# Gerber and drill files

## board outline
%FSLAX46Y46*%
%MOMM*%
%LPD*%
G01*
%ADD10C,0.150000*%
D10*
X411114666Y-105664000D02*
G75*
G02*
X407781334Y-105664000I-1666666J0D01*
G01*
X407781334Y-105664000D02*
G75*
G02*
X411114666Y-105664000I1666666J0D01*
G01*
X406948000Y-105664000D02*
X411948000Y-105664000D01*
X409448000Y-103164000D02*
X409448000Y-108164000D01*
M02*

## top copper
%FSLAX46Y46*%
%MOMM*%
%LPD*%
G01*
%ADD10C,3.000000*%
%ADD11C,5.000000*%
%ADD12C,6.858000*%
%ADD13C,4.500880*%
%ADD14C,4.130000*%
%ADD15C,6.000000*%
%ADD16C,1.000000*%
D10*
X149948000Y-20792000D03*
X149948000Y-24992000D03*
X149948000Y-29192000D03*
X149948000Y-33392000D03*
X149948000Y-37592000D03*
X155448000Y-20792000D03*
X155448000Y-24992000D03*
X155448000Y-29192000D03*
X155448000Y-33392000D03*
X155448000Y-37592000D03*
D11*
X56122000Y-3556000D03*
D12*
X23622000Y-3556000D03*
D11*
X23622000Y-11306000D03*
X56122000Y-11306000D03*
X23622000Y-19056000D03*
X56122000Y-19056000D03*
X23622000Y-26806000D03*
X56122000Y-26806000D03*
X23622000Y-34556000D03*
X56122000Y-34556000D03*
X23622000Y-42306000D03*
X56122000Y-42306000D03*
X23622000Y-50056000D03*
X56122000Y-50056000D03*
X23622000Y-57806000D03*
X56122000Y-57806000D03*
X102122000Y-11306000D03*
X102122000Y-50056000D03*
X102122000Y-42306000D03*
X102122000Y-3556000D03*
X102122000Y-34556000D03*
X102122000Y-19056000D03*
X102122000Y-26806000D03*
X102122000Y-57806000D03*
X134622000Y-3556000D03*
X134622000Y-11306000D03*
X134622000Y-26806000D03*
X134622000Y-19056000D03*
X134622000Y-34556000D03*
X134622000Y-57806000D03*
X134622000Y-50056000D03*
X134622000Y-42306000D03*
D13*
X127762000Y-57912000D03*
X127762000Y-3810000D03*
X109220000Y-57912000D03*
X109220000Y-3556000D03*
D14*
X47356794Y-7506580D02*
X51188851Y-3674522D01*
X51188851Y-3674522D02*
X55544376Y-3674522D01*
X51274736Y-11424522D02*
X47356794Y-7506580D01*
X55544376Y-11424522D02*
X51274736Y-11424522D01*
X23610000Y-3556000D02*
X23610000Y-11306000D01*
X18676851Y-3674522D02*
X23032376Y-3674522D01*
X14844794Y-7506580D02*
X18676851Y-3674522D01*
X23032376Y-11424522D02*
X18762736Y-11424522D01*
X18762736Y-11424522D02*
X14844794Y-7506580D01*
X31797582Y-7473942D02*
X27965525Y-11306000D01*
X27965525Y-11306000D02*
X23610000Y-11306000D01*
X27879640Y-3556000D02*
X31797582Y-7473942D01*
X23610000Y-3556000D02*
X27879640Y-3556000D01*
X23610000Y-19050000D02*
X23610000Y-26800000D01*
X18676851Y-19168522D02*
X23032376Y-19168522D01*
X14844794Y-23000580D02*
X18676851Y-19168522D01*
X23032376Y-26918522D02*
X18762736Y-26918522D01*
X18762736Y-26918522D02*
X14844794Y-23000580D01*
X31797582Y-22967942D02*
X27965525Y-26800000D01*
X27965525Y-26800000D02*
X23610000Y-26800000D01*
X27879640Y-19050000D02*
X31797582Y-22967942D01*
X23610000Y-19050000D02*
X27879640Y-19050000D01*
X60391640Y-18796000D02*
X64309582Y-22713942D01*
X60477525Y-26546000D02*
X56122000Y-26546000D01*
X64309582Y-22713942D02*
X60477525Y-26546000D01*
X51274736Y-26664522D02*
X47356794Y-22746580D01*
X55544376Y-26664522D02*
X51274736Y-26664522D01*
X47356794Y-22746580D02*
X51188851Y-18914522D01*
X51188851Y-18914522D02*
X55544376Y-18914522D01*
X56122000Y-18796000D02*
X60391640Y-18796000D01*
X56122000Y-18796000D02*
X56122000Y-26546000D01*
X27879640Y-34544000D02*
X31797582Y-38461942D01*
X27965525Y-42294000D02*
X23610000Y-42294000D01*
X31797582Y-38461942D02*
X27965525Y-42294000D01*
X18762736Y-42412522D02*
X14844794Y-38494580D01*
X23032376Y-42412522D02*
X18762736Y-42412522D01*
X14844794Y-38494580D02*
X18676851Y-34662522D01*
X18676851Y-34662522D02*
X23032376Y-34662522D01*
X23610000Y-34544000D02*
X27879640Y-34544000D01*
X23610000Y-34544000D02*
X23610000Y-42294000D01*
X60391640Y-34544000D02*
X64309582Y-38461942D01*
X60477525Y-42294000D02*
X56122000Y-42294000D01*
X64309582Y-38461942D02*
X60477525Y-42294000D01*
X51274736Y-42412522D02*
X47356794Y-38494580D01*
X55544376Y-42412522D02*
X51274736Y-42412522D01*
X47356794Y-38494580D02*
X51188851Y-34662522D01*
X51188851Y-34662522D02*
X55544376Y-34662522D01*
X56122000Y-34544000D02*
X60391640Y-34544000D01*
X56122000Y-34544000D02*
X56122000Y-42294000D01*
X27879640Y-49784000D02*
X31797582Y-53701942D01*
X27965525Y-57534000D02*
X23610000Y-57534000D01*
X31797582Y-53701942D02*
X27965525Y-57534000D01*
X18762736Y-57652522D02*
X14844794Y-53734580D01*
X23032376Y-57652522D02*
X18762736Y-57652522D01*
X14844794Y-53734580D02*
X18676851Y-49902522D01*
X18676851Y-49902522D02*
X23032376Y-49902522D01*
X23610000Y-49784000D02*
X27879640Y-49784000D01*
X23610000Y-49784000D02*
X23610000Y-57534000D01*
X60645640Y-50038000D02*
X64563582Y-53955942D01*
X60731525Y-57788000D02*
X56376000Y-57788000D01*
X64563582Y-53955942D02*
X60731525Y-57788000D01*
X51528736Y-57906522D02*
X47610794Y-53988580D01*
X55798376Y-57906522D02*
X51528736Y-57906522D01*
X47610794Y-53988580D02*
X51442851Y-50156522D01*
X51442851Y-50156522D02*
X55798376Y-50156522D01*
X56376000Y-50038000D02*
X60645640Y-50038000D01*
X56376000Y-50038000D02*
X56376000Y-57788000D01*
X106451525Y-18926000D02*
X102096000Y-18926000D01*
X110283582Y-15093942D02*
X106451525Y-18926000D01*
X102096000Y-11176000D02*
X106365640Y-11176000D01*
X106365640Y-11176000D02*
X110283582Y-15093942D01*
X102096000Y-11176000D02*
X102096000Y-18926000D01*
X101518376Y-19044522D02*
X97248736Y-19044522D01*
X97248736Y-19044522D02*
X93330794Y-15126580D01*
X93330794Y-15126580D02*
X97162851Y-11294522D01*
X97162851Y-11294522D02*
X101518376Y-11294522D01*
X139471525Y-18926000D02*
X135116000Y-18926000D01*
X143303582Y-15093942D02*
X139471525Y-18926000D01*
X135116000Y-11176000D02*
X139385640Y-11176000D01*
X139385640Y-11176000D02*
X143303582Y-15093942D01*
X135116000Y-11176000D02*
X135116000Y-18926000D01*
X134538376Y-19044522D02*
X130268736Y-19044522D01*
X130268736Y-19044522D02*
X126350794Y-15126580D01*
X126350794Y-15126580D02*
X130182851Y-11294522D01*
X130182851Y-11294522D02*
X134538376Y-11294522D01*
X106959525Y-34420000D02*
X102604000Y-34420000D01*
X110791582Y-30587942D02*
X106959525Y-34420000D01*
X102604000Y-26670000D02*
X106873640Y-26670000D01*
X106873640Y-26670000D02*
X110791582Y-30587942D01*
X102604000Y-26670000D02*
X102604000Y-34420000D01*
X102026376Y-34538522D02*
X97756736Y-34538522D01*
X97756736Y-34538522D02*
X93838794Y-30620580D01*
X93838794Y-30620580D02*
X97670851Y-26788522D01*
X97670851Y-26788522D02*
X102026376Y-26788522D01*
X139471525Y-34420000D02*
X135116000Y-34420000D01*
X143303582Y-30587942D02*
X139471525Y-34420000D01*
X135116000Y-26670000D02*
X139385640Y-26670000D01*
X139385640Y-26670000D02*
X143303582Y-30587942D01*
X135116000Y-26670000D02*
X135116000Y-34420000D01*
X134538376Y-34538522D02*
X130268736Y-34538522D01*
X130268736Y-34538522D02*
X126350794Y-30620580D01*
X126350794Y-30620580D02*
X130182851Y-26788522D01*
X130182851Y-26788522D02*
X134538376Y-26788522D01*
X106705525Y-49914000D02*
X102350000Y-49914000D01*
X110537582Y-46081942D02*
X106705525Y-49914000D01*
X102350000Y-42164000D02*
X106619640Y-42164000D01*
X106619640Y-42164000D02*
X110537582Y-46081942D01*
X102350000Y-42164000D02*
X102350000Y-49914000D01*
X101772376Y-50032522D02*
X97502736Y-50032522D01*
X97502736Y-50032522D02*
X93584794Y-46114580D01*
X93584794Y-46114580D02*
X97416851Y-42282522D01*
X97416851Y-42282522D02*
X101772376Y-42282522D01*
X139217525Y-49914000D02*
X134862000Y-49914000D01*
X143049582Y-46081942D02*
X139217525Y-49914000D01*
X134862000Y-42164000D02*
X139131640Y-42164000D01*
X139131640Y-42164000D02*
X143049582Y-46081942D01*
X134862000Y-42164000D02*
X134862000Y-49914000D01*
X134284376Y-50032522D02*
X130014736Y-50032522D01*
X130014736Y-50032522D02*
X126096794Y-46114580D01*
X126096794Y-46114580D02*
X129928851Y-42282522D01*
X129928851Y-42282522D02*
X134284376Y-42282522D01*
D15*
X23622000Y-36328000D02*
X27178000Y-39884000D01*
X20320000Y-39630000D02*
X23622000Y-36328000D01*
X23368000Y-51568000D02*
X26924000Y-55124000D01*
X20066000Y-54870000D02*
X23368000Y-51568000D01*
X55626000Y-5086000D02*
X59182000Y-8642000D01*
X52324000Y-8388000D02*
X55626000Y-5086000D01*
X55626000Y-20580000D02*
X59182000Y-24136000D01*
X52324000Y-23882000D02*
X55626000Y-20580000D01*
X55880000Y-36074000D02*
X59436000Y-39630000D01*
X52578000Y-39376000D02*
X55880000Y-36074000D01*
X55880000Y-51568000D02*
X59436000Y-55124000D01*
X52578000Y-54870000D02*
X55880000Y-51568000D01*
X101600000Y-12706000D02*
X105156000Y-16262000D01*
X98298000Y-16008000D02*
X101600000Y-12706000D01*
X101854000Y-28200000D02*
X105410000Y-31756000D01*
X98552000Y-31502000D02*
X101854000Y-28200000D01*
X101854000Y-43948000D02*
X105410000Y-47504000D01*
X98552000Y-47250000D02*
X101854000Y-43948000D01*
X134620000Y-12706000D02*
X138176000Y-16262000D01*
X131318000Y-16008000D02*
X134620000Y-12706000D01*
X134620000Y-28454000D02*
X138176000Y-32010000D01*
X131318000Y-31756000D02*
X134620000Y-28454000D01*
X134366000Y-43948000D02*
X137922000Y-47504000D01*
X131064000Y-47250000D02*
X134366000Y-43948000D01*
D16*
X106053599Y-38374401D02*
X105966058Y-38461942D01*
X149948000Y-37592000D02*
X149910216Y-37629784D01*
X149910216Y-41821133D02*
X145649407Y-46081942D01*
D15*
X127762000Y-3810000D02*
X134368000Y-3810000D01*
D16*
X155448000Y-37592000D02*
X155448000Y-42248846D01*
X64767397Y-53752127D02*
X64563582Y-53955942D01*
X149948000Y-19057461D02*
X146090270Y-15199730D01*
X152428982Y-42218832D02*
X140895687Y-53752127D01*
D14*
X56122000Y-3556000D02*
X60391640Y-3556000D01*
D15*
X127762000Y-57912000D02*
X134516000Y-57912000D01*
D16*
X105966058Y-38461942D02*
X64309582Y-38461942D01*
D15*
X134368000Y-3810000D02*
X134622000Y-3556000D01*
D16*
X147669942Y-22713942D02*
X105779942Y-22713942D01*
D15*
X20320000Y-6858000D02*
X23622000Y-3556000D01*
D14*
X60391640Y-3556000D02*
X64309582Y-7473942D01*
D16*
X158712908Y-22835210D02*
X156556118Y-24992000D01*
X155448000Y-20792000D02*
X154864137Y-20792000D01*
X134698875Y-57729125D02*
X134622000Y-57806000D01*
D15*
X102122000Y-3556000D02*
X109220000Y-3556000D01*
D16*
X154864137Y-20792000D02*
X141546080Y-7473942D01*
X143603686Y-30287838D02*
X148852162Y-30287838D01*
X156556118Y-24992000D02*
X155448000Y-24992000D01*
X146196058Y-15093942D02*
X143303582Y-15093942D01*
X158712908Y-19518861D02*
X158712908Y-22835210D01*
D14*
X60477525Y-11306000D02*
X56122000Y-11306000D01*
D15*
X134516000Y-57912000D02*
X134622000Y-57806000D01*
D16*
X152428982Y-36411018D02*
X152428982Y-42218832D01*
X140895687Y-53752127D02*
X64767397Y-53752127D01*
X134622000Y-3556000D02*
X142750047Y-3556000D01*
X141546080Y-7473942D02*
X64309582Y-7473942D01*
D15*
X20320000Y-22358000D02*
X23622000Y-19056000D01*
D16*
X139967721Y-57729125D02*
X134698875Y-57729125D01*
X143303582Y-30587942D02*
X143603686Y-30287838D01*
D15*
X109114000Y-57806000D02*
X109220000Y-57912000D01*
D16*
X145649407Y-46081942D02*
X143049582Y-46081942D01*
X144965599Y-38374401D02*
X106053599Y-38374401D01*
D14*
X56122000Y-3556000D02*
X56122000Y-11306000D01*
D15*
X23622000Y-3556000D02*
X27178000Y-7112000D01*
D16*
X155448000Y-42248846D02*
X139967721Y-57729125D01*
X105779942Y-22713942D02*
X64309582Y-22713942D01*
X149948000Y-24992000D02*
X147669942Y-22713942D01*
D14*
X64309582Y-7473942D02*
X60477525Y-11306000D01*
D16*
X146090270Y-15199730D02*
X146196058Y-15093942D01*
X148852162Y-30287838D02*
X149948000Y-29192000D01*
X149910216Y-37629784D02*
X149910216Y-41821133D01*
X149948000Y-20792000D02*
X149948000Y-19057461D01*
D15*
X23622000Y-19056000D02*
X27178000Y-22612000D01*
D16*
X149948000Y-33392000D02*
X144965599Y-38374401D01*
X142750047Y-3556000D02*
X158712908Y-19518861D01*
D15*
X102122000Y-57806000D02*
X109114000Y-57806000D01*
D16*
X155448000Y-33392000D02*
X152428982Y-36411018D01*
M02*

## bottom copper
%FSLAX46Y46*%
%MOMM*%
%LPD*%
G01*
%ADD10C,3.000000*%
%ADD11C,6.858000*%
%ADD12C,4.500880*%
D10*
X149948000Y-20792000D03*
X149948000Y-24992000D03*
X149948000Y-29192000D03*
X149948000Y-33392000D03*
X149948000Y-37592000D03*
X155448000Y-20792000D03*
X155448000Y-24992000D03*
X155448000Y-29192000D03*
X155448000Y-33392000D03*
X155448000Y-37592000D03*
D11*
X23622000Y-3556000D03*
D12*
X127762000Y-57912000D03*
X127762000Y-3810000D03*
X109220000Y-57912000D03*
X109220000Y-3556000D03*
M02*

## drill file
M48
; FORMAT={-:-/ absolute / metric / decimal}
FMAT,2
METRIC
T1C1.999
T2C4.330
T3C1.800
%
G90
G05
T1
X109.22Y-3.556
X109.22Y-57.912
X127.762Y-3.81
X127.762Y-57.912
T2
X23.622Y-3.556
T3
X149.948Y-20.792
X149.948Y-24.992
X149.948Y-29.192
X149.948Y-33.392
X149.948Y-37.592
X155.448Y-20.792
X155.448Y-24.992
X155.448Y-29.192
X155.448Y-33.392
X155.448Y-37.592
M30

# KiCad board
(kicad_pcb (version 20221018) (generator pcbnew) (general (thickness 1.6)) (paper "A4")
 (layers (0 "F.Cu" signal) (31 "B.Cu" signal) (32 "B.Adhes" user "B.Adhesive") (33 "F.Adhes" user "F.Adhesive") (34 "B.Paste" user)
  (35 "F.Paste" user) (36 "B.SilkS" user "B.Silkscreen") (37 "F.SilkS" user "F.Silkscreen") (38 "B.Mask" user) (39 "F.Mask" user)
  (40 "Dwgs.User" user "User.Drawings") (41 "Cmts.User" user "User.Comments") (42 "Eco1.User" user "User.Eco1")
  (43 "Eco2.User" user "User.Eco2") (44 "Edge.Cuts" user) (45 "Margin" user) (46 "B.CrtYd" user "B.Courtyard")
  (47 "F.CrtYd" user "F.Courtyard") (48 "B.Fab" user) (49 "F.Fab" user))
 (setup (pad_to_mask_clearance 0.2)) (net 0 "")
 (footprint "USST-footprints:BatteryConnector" (layer "F.Cu") (at 149.948 37.592)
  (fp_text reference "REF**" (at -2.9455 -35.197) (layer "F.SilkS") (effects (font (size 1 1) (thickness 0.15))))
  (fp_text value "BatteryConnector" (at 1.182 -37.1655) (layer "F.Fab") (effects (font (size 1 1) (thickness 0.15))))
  (pad "" np_thru_hole circle (at 0 -16.8) (size 3 3) (drill 1.8) (layers "*.Cu"))
  (pad "" np_thru_hole circle (at 0 -12.6) (size 3 3) (drill 1.8) (layers "*.Cu"))
  (pad "" np_thru_hole circle (at 0 -8.4) (size 3 3) (drill 1.8) (layers "*.Cu"))
  (pad "" np_thru_hole circle (at 0 -4.2) (size 3 3) (drill 1.8) (layers "*.Cu"))
  (pad "" np_thru_hole circle (at 0 0) (size 3 3) (drill 1.8) (layers "*.Cu"))
  (pad "" np_thru_hole circle (at 5.5 -16.8) (size 3 3) (drill 1.8) (layers "*.Cu"))
  (pad "" np_thru_hole circle (at 5.5 -12.6) (size 3 3) (drill 1.8) (layers "*.Cu"))
  (pad "" np_thru_hole circle (at 5.5 -8.4) (size 3 3) (drill 1.8) (layers "*.Cu"))
  (pad "" np_thru_hole circle (at 5.5 -4.2) (size 3 3) (drill 1.8) (layers "*.Cu"))
  (pad "" np_thru_hole circle (at 5.5 0) (size 3 3) (drill 1.8) (layers "*.Cu")))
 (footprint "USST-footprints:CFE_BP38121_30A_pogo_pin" (layer "F.Cu") (at 96 14.986)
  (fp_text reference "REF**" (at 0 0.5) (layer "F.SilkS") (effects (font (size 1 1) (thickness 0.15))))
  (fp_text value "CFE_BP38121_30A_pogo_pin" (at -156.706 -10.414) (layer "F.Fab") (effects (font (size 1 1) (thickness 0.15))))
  (pad "1" smd circle (at -39.878 -11.43) (size 5 5) (layers "F.Cu" "F.Paste" "F.Mask")))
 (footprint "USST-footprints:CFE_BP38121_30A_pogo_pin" (layer "F.Cu") (at 63.5 14.986)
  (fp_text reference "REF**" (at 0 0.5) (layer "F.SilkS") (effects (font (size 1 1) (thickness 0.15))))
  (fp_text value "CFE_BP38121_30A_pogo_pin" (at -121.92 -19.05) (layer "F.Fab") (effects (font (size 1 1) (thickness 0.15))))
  (pad "1" thru_hole circle (at -39.878 -11.43) (size 6.858 6.858) (drill 4.33) (layers "*.Cu" "*.Mask")))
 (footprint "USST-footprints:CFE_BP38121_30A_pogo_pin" (layer "F.Cu") (at 63.5 22.736)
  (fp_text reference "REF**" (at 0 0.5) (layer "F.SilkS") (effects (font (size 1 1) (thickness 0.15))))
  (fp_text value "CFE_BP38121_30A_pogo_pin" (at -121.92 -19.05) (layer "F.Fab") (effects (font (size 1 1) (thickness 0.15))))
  (pad "2" smd circle (at -39.878 -11.43) (size 5 5) (layers "F.Cu" "F.Paste" "F.Mask")))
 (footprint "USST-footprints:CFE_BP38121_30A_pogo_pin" (layer "F.Cu") (at 96 22.736)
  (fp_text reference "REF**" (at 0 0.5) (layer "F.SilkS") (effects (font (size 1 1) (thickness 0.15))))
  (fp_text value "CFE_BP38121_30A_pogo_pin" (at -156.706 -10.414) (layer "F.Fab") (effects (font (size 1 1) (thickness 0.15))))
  (pad "2" smd circle (at -39.878 -11.43) (size 5 5) (layers "F.Cu" "F.Paste" "F.Mask")))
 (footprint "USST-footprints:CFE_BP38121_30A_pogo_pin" (layer "F.Cu") (at 63.5 30.486)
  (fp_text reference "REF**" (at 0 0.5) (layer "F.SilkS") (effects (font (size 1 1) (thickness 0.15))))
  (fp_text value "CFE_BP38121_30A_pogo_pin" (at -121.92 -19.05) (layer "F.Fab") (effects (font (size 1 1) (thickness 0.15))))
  (pad "3" smd circle (at -39.878 -11.43) (size 5 5) (layers "F.Cu" "F.Paste" "F.Mask")))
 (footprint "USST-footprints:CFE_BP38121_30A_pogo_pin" (layer "F.Cu") (at 96 30.486)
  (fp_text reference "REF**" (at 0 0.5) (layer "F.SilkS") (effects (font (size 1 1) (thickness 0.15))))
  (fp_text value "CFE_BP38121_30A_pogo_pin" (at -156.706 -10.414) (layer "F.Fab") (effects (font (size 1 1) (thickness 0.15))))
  (pad "3" smd circle (at -39.878 -11.43) (size 5 5) (layers "F.Cu" "F.Paste" "F.Mask")))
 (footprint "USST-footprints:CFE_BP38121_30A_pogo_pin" (layer "F.Cu") (at 63.5 38.236)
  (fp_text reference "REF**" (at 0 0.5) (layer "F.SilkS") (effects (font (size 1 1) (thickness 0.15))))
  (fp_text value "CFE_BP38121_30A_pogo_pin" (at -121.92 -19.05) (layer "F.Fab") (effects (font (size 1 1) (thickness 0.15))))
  (pad "4" smd circle (at -39.878 -11.43) (size 5 5) (layers "F.Cu" "F.Paste" "F.Mask")))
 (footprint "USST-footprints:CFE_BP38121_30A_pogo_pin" (layer "F.Cu") (at 96 38.236)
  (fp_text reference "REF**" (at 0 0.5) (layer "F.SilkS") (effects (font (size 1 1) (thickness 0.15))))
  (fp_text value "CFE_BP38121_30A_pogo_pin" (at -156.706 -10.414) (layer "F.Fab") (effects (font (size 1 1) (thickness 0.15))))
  (pad "4" smd circle (at -39.878 -11.43) (size 5 5) (layers "F.Cu" "F.Paste" "F.Mask")))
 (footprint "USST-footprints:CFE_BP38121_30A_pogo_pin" (layer "F.Cu") (at 63.5 45.986)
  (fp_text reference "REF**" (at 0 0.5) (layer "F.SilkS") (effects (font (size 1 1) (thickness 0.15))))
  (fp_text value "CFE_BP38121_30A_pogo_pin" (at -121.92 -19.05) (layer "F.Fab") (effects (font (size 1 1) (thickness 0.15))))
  (pad "5" smd circle (at -39.878 -11.43) (size 5 5) (layers "F.Cu" "F.Paste" "F.Mask")))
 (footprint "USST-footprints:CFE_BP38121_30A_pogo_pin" (layer "F.Cu") (at 96 45.986)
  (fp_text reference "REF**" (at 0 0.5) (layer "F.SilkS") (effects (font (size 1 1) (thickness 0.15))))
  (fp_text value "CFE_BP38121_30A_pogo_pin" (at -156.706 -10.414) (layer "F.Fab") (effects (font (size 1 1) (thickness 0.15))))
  (pad "5" smd circle (at -39.878 -11.43) (size 5 5) (layers "F.Cu" "F.Paste" "F.Mask")))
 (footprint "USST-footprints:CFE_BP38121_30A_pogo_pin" (layer "F.Cu") (at 63.5 53.736)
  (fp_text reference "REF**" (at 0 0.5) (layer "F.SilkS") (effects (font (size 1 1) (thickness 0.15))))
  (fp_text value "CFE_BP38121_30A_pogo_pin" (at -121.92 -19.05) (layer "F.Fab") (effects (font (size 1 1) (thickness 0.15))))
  (pad "6" smd circle (at -39.878 -11.43) (size 5 5) (layers "F.Cu" "F.Paste" "F.Mask")))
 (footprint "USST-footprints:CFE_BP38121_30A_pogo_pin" (layer "F.Cu") (at 96 53.736)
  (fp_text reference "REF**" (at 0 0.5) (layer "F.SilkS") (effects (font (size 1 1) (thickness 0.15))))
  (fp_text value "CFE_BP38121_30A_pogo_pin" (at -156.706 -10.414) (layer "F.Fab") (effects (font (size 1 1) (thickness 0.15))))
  (pad "6" smd circle (at -39.878 -11.43) (size 5 5) (layers "F.Cu" "F.Paste" "F.Mask")))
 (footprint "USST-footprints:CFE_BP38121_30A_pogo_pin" (layer "F.Cu") (at 63.5 61.486)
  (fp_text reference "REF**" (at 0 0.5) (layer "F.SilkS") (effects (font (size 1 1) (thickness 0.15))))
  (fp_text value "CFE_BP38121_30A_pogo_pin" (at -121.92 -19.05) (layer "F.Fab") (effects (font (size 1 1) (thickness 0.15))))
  (pad "7" smd circle (at -39.878 -11.43) (size 5 5) (layers "F.Cu" "F.Paste" "F.Mask")))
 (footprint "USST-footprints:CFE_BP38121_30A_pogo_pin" (layer "F.Cu") (at 96 61.486)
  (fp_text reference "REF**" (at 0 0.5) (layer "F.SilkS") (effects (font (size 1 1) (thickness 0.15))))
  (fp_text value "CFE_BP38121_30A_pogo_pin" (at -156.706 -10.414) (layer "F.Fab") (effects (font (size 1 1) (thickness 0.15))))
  (pad "7" smd circle (at -39.878 -11.43) (size 5 5) (layers "F.Cu" "F.Paste" "F.Mask")))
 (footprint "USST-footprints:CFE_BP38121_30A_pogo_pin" (layer "F.Cu") (at 63.5 69.236)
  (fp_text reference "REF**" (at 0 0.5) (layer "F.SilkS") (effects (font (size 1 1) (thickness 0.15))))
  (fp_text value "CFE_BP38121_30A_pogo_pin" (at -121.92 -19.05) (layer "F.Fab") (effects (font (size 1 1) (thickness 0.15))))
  (pad "8" smd circle (at -39.878 -11.43) (size 5 5) (layers "F.Cu" "F.Paste" "F.Mask")))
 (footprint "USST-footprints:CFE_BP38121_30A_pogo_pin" (layer "F.Cu") (at 96 69.236)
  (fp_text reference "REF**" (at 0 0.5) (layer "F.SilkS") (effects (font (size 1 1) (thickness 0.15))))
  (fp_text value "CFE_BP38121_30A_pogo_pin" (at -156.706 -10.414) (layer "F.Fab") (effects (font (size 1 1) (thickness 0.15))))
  (pad "8" smd circle (at -39.878 -11.43) (size 5 5) (layers "F.Cu" "F.Paste" "F.Mask")))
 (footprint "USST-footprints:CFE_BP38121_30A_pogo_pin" (layer "F.Cu") (at 142 22.736)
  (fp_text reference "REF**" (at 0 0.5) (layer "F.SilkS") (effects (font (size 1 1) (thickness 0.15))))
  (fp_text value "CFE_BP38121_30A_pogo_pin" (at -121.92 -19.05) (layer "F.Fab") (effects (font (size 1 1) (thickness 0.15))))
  (pad "2" smd circle (at -39.878 -11.43) (size 5 5) (layers "F.Cu" "F.Paste" "F.Mask")))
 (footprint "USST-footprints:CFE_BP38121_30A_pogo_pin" (layer "F.Cu") (at 142 61.486)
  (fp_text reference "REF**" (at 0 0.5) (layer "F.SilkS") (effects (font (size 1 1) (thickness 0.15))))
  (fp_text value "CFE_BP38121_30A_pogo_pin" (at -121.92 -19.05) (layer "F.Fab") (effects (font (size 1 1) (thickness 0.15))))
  (pad "7" smd circle (at -39.878 -11.43) (size 5 5) (layers "F.Cu" "F.Paste" "F.Mask")))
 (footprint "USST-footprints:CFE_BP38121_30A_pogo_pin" (layer "F.Cu") (at 142 53.736)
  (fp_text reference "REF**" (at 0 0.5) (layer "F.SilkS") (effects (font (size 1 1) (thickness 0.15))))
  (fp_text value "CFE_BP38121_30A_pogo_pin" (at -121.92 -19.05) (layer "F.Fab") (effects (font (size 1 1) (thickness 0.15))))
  (pad "6" smd circle (at -39.878 -11.43) (size 5 5) (layers "F.Cu" "F.Paste" "F.Mask")))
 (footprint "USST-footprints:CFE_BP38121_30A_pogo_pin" (layer "F.Cu") (at 142 14.986)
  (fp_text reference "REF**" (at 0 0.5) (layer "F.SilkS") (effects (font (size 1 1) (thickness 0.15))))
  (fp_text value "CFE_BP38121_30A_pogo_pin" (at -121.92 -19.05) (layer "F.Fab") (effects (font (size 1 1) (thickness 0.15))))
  (pad "1" smd circle (at -39.878 -11.43) (size 5 5) (layers "F.Cu" "F.Paste" "F.Mask")))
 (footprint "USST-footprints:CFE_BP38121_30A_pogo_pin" (layer "F.Cu") (at 142 45.986)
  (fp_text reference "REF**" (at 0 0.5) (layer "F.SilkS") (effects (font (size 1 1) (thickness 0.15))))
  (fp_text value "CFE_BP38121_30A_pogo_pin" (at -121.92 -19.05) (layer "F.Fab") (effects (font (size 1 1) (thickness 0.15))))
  (pad "5" smd circle (at -39.878 -11.43) (size 5 5) (layers "F.Cu" "F.Paste" "F.Mask")))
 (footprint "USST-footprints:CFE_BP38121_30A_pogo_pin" (layer "F.Cu") (at 142 30.486)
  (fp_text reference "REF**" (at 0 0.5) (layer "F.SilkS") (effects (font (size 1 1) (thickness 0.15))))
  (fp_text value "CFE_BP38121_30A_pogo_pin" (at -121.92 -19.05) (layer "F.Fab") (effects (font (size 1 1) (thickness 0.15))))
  (pad "3" smd circle (at -39.878 -11.43) (size 5 5) (layers "F.Cu" "F.Paste" "F.Mask")))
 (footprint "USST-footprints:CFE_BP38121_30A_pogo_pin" (layer "F.Cu") (at 142 38.236)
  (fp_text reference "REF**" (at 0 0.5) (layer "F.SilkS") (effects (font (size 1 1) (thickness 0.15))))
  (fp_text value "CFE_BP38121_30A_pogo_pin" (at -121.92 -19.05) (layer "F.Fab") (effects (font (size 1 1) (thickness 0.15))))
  (pad "4" smd circle (at -39.878 -11.43) (size 5 5) (layers "F.Cu" "F.Paste" "F.Mask")))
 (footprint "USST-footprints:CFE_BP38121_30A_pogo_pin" (layer "F.Cu") (at 142 69.236)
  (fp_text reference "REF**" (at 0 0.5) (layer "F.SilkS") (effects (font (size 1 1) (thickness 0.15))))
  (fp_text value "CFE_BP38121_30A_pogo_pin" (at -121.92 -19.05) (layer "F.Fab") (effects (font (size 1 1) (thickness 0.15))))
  (pad "8" smd circle (at -39.878 -11.43) (size 5 5) (layers "F.Cu" "F.Paste" "F.Mask")))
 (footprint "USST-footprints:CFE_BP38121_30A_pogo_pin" (layer "F.Cu") (at 174.5 14.986)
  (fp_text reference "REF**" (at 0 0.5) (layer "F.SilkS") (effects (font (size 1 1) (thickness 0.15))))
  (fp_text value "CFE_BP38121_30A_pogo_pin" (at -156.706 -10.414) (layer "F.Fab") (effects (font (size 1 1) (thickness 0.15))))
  (pad "1" smd circle (at -39.878 -11.43) (size 5 5) (layers "F.Cu" "F.Paste" "F.Mask")))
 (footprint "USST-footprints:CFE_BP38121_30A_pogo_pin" (layer "F.Cu") (at 174.5 22.736)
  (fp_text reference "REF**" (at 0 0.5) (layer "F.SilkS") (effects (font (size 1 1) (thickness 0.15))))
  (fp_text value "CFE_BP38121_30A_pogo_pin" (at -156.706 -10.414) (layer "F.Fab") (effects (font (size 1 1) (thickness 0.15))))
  (pad "2" smd circle (at -39.878 -11.43) (size 5 5) (layers "F.Cu" "F.Paste" "F.Mask")))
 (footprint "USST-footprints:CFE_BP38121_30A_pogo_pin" (layer "F.Cu") (at 174.5 38.236)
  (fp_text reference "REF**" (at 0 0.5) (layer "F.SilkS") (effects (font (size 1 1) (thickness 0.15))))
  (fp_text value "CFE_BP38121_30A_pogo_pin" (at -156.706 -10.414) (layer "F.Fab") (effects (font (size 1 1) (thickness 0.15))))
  (pad "4" smd circle (at -39.878 -11.43) (size 5 5) (layers "F.Cu" "F.Paste" "F.Mask")))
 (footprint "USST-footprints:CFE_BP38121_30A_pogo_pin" (layer "F.Cu") (at 174.5 30.486)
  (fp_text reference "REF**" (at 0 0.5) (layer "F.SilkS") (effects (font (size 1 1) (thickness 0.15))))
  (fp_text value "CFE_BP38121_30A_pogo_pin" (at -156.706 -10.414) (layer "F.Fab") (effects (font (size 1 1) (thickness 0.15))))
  (pad "3" smd circle (at -39.878 -11.43) (size 5 5) (layers "F.Cu" "F.Paste" "F.Mask")))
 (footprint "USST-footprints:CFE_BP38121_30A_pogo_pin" (layer "F.Cu") (at 174.5 45.986)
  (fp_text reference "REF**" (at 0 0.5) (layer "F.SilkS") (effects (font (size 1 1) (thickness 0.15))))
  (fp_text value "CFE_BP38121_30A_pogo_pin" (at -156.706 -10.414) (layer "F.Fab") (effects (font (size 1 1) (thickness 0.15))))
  (pad "5" smd circle (at -39.878 -11.43) (size 5 5) (layers "F.Cu" "F.Paste" "F.Mask")))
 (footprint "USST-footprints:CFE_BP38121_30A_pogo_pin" (layer "F.Cu") (at 174.5 69.236)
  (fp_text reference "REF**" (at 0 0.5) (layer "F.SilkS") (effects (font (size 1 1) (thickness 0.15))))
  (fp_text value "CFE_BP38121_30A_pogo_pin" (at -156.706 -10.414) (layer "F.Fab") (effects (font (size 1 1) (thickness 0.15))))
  (pad "8" smd circle (at -39.878 -11.43) (size 5 5) (layers "F.Cu" "F.Paste" "F.Mask")))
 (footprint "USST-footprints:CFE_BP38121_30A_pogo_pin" (layer "F.Cu") (at 174.5 61.486)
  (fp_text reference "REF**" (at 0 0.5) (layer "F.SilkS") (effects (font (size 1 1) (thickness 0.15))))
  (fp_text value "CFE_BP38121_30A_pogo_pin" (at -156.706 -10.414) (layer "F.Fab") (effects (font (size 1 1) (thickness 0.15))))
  (pad "7" smd circle (at -39.878 -11.43) (size 5 5) (layers "F.Cu" "F.Paste" "F.Mask")))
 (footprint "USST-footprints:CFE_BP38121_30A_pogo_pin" (layer "F.Cu") (at 174.5 53.736)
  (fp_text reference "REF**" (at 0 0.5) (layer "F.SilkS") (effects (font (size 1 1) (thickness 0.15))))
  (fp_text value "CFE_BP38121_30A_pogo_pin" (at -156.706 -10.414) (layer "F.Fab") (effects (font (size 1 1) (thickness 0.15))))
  (pad "6" smd circle (at -39.878 -11.43) (size 5 5) (layers "F.Cu" "F.Paste" "F.Mask")))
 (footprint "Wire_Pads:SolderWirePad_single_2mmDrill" (layer "F.Cu") (at 127.762 57.912)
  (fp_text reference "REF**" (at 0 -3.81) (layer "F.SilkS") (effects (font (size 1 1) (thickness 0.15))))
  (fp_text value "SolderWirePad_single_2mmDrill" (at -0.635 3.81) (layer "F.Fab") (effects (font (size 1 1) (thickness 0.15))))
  (pad "1" thru_hole circle (at 0 0) (size 4.50088 4.50088) (drill 1.99898) (layers "*.Cu" "*.Mask")))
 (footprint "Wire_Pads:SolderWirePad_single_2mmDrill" (layer "F.Cu") (at 127.762 3.81)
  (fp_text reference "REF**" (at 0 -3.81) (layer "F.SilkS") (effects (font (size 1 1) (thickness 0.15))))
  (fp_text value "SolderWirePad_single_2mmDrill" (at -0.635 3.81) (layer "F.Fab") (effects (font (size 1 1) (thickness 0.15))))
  (pad "1" thru_hole circle (at 0 0) (size 4.50088 4.50088) (drill 1.99898) (layers "*.Cu" "*.Mask")))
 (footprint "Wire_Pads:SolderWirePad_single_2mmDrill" (layer "F.Cu") (at 109.22 57.912)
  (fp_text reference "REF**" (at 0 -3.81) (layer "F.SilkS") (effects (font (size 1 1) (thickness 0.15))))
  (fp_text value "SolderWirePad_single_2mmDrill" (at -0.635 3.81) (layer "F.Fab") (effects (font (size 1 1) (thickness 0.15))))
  (pad "1" thru_hole circle (at 0 0) (size 4.50088 4.50088) (drill 1.99898) (layers "*.Cu" "*.Mask")))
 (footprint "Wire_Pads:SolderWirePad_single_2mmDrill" (layer "F.Cu") (at 109.22 3.556)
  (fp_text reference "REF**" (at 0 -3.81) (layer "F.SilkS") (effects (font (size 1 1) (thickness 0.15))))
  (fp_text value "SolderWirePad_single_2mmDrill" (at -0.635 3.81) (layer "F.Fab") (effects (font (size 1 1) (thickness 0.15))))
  (pad "1" thru_hole circle (at 0 0) (size 4.50088 4.50088) (drill 1.99898) (layers "*.Cu" "*.Mask")))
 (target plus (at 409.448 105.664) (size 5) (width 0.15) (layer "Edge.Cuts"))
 (segment (start 47.356794 7.50658) (end 51.188851 3.674522) (width 4.13) (layer "F.Cu") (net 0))
 (segment (start 51.188851 3.674522) (end 55.544376 3.674522) (width 4.13) (layer "F.Cu") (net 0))
 (segment (start 51.274736 11.424522) (end 47.356794 7.50658) (width 4.13) (layer "F.Cu") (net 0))
 (segment (start 55.544376 11.424522) (end 51.274736 11.424522) (width 4.13) (layer "F.Cu") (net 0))
 (segment (start 23.61 3.556) (end 23.61 11.306) (width 4.13) (layer "F.Cu") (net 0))
 (segment (start 18.676851 3.674522) (end 23.032376 3.674522) (width 4.13) (layer "F.Cu") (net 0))
 (segment (start 14.844794 7.50658) (end 18.676851 3.674522) (width 4.13) (layer "F.Cu") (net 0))
 (segment (start 23.032376 11.424522) (end 18.762736 11.424522) (width 4.13) (layer "F.Cu") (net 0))
 (segment (start 18.762736 11.424522) (end 14.844794 7.50658) (width 4.13) (layer "F.Cu") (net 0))
 (segment (start 31.797582 7.473942) (end 27.965525 11.306) (width 4.13) (layer "F.Cu") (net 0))
 (segment (start 27.965525 11.306) (end 23.61 11.306) (width 4.13) (layer "F.Cu") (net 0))
 (segment (start 27.87964 3.556) (end 31.797582 7.473942) (width 4.13) (layer "F.Cu") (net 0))
 (segment (start 23.61 3.556) (end 27.87964 3.556) (width 4.13) (layer "F.Cu") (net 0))
 (segment (start 23.61 19.05) (end 23.61 26.8) (width 4.13) (layer "F.Cu") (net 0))
 (segment (start 18.676851 19.168522) (end 23.032376 19.168522) (width 4.13) (layer "F.Cu") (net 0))
 (segment (start 14.844794 23.00058) (end 18.676851 19.168522) (width 4.13) (layer "F.Cu") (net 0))
 (segment (start 23.032376 26.918522) (end 18.762736 26.918522) (width 4.13) (layer "F.Cu") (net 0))
 (segment (start 18.762736 26.918522) (end 14.844794 23.00058) (width 4.13) (layer "F.Cu") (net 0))
 (segment (start 31.797582 22.967942) (end 27.965525 26.8) (width 4.13) (layer "F.Cu") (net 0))
 (segment (start 27.965525 26.8) (end 23.61 26.8) (width 4.13) (layer "F.Cu") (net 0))
 (segment (start 27.87964 19.05) (end 31.797582 22.967942) (width 4.13) (layer "F.Cu") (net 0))
 (segment (start 23.61 19.05) (end 27.87964 19.05) (width 4.13) (layer "F.Cu") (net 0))
 (segment (start 60.39164 18.796) (end 64.309582 22.713942) (width 4.13) (layer "F.Cu") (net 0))
 (segment (start 60.477525 26.546) (end 56.122 26.546) (width 4.13) (layer "F.Cu") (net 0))
 (segment (start 64.309582 22.713942) (end 60.477525 26.546) (width 4.13) (layer "F.Cu") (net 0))
 (segment (start 51.274736 26.664522) (end 47.356794 22.74658) (width 4.13) (layer "F.Cu") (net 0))
 (segment (start 55.544376 26.664522) (end 51.274736 26.664522) (width 4.13) (layer "F.Cu") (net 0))
 (segment (start 47.356794 22.74658) (end 51.188851 18.914522) (width 4.13) (layer "F.Cu") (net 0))
 (segment (start 51.188851 18.914522) (end 55.544376 18.914522) (width 4.13) (layer "F.Cu") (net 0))
 (segment (start 56.122 18.796) (end 60.39164 18.796) (width 4.13) (layer "F.Cu") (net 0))
 (segment (start 56.122 18.796) (end 56.122 26.546) (width 4.13) (layer "F.Cu") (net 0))
 (segment (start 27.87964 34.544) (end 31.797582 38.461942) (width 4.13) (layer "F.Cu") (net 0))
 (segment (start 27.965525 42.294) (end 23.61 42.294) (width 4.13) (layer "F.Cu") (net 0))
 (segment (start 31.797582 38.461942) (end 27.965525 42.294) (width 4.13) (layer "F.Cu") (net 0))
 (segment (start 18.762736 42.412522) (end 14.844794 38.49458) (width 4.13) (layer "F.Cu") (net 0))
 (segment (start 23.032376 42.412522) (end 18.762736 42.412522) (width 4.13) (layer "F.Cu") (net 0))
 (segment (start 14.844794 38.49458) (end 18.676851 34.662522) (width 4.13) (layer "F.Cu") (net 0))
 (segment (start 18.676851 34.662522) (end 23.032376 34.662522) (width 4.13) (layer "F.Cu") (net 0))
 (segment (start 23.61 34.544) (end 27.87964 34.544) (width 4.13) (layer "F.Cu") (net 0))
 (segment (start 23.61 34.544) (end 23.61 42.294) (width 4.13) (layer "F.Cu") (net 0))
 (segment (start 60.39164 34.544) (end 64.309582 38.461942) (width 4.13) (layer "F.Cu") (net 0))
 (segment (start 60.477525 42.294) (end 56.122 42.294) (width 4.13) (layer "F.Cu") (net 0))
 (segment (start 64.309582 38.461942) (end 60.477525 42.294) (width 4.13) (layer "F.Cu") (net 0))
 (segment (start 51.274736 42.412522) (end 47.356794 38.49458) (width 4.13) (layer "F.Cu") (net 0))
 (segment (start 55.544376 42.412522) (end 51.274736 42.412522) (width 4.13) (layer "F.Cu") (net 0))
 (segment (start 47.356794 38.49458) (end 51.188851 34.662522) (width 4.13) (layer "F.Cu") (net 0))
 (segment (start 51.188851 34.662522) (end 55.544376 34.662522) (width 4.13) (layer "F.Cu") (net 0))
 (segment (start 56.122 34.544) (end 60.39164 34.544) (width 4.13) (layer "F.Cu") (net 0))
 (segment (start 56.122 34.544) (end 56.122 42.294) (width 4.13) (layer "F.Cu") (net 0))
 (segment (start 27.87964 49.784) (end 31.797582 53.701942) (width 4.13) (layer "F.Cu") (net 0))
 (segment (start 27.965525 57.534) (end 23.61 57.534) (width 4.13) (layer "F.Cu") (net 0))
 (segment (start 31.797582 53.701942) (end 27.965525 57.534) (width 4.13) (layer "F.Cu") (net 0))
 (segment (start 18.762736 57.652522) (end 14.844794 53.73458) (width 4.13) (layer "F.Cu") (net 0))
 (segment (start 23.032376 57.652522) (end 18.762736 57.652522) (width 4.13) (layer "F.Cu") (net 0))
 (segment (start 14.844794 53.73458) (end 18.676851 49.902522) (width 4.13) (layer "F.Cu") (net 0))
 (segment (start 18.676851 49.902522) (end 23.032376 49.902522) (width 4.13) (layer "F.Cu") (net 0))
 (segment (start 23.61 49.784) (end 27.87964 49.784) (width 4.13) (layer "F.Cu") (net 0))
 (segment (start 23.61 49.784) (end 23.61 57.534) (width 4.13) (layer "F.Cu") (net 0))
 (segment (start 60.64564 50.038) (end 64.563582 53.955942) (width 4.13) (layer "F.Cu") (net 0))
 (segment (start 60.731525 57.788) (end 56.376 57.788) (width 4.13) (layer "F.Cu") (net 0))
 (segment (start 64.563582 53.955942) (end 60.731525 57.788) (width 4.13) (layer "F.Cu") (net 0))
 (segment (start 51.528736 57.906522) (end 47.610794 53.98858) (width 4.13) (layer "F.Cu") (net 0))
 (segment (start 55.798376 57.906522) (end 51.528736 57.906522) (width 4.13) (layer "F.Cu") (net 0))
 (segment (start 47.610794 53.98858) (end 51.442851 50.156522) (width 4.13) (layer "F.Cu") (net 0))
 (segment (start 51.442851 50.156522) (end 55.798376 50.156522) (width 4.13) (layer "F.Cu") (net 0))
 (segment (start 56.376 50.038) (end 60.64564 50.038) (width 4.13) (layer "F.Cu") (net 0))
 (segment (start 56.376 50.038) (end 56.376 57.788) (width 4.13) (layer "F.Cu") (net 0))
 (segment (start 106.451525 18.926) (end 102.096 18.926) (width 4.13) (layer "F.Cu") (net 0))
 (segment (start 110.283582 15.093942) (end 106.451525 18.926) (width 4.13) (layer "F.Cu") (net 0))
 (segment (start 102.096 11.176) (end 106.36564 11.176) (width 4.13) (layer "F.Cu") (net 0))
 (segment (start 106.36564 11.176) (end 110.283582 15.093942) (width 4.13) (layer "F.Cu") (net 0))
 (segment (start 102.096 11.176) (end 102.096 18.926) (width 4.13) (layer "F.Cu") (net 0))
 (segment (start 101.518376 19.044522) (end 97.248736 19.044522) (width 4.13) (layer "F.Cu") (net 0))
 (segment (start 97.248736 19.044522) (end 93.330794 15.12658) (width 4.13) (layer "F.Cu") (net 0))
 (segment (start 93.330794 15.12658) (end 97.162851 11.294522) (width 4.13) (layer "F.Cu") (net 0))
 (segment (start 97.162851 11.294522) (end 101.518376 11.294522) (width 4.13) (layer "F.Cu") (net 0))
 (segment (start 139.471525 18.926) (end 135.116 18.926) (width 4.13) (layer "F.Cu") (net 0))
 (segment (start 143.303582 15.093942) (end 139.471525 18.926) (width 4.13) (layer "F.Cu") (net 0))
 (segment (start 135.116 11.176) (end 139.38564 11.176) (width 4.13) (layer "F.Cu") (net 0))
 (segment (start 139.38564 11.176) (end 143.303582 15.093942) (width 4.13) (layer "F.Cu") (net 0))
 (segment (start 135.116 11.176) (end 135.116 18.926) (width 4.13) (layer "F.Cu") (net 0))
 (segment (start 134.538376 19.044522) (end 130.268736 19.044522) (width 4.13) (layer "F.Cu") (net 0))
 (segment (start 130.268736 19.044522) (end 126.350794 15.12658) (width 4.13) (layer "F.Cu") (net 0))
 (segment (start 126.350794 15.12658) (end 130.182851 11.294522) (width 4.13) (layer "F.Cu") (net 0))
 (segment (start 130.182851 11.294522) (end 134.538376 11.294522) (width 4.13) (layer "F.Cu") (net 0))
 (segment (start 106.959525 34.42) (end 102.604 34.42) (width 4.13) (layer "F.Cu") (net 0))
 (segment (start 110.791582 30.587942) (end 106.959525 34.42) (width 4.13) (layer "F.Cu") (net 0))
 (segment (start 102.604 26.67) (end 106.87364 26.67) (width 4.13) (layer "F.Cu") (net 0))
 (segment (start 106.87364 26.67) (end 110.791582 30.587942) (width 4.13) (layer "F.Cu") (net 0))
 (segment (start 102.604 26.67) (end 102.604 34.42) (width 4.13) (layer "F.Cu") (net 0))
 (segment (start 102.026376 34.538522) (end 97.756736 34.538522) (width 4.13) (layer "F.Cu") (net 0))
 (segment (start 97.756736 34.538522) (end 93.838794 30.62058) (width 4.13) (layer "F.Cu") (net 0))
 (segment (start 93.838794 30.62058) (end 97.670851 26.788522) (width 4.13) (layer "F.Cu") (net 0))
 (segment (start 97.670851 26.788522) (end 102.026376 26.788522) (width 4.13) (layer "F.Cu") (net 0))
 (segment (start 139.471525 34.42) (end 135.116 34.42) (width 4.13) (layer "F.Cu") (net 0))
 (segment (start 143.303582 30.587942) (end 139.471525 34.42) (width 4.13) (layer "F.Cu") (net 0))
 (segment (start 135.116 26.67) (end 139.38564 26.67) (width 4.13) (layer "F.Cu") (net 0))
 (segment (start 139.38564 26.67) (end 143.303582 30.587942) (width 4.13) (layer "F.Cu") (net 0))
 (segment (start 135.116 26.67) (end 135.116 34.42) (width 4.13) (layer "F.Cu") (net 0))
 (segment (start 134.538376 34.538522) (end 130.268736 34.538522) (width 4.13) (layer "F.Cu") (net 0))
 (segment (start 130.268736 34.538522) (end 126.350794 30.62058) (width 4.13) (layer "F.Cu") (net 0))
 (segment (start 126.350794 30.62058) (end 130.182851 26.788522) (width 4.13) (layer "F.Cu") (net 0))
 (segment (start 130.182851 26.788522) (end 134.538376 26.788522) (width 4.13) (layer "F.Cu") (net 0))
 (segment (start 106.705525 49.914) (end 102.35 49.914) (width 4.13) (layer "F.Cu") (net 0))
 (segment (start 110.537582 46.081942) (end 106.705525 49.914) (width 4.13) (layer "F.Cu") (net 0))
 (segment (start 102.35 42.164) (end 106.61964 42.164) (width 4.13) (layer "F.Cu") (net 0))
 (segment (start 106.61964 42.164) (end 110.537582 46.081942) (width 4.13) (layer "F.Cu") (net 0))
 (segment (start 102.35 42.164) (end 102.35 49.914) (width 4.13) (layer "F.Cu") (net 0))
 (segment (start 101.772376 50.032522) (end 97.502736 50.032522) (width 4.13) (layer "F.Cu") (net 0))
 (segment (start 97.502736 50.032522) (end 93.584794 46.11458) (width 4.13) (layer "F.Cu") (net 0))
 (segment (start 93.584794 46.11458) (end 97.416851 42.282522) (width 4.13) (layer "F.Cu") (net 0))
 (segment (start 97.416851 42.282522) (end 101.772376 42.282522) (width 4.13) (layer "F.Cu") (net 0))
 (segment (start 139.217525 49.914) (end 134.862 49.914) (width 4.13) (layer "F.Cu") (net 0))
 (segment (start 143.049582 46.081942) (end 139.217525 49.914) (width 4.13) (layer "F.Cu") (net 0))
 (segment (start 134.862 42.164) (end 139.13164 42.164) (width 4.13) (layer "F.Cu") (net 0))
 (segment (start 139.13164 42.164) (end 143.049582 46.081942) (width 4.13) (layer "F.Cu") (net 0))
 (segment (start 134.862 42.164) (end 134.862 49.914) (width 4.13) (layer "F.Cu") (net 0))
 (segment (start 134.284376 50.032522) (end 130.014736 50.032522) (width 4.13) (layer "F.Cu") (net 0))
 (segment (start 130.014736 50.032522) (end 126.096794 46.11458) (width 4.13) (layer "F.Cu") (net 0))
 (segment (start 126.096794 46.11458) (end 129.928851 42.282522) (width 4.13) (layer "F.Cu") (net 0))
 (segment (start 129.928851 42.282522) (end 134.284376 42.282522) (width 4.13) (layer "F.Cu") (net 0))
 (segment (start 23.622 36.328) (end 27.178 39.884) (width 6) (layer "F.Cu") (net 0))
 (segment (start 20.32 39.63) (end 23.622 36.328) (width 6) (layer "F.Cu") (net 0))
 (segment (start 23.368 51.568) (end 26.924 55.124) (width 6) (layer "F.Cu") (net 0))
 (segment (start 20.066 54.87) (end 23.368 51.568) (width 6) (layer "F.Cu") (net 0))
 (segment (start 55.626 5.086) (end 59.182 8.642) (width 6) (layer "F.Cu") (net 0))
 (segment (start 52.324 8.388) (end 55.626 5.086) (width 6) (layer "F.Cu") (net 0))
 (segment (start 55.626 20.58) (end 59.182 24.136) (width 6) (layer "F.Cu") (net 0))
 (segment (start 52.324 23.882) (end 55.626 20.58) (width 6) (layer "F.Cu") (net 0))
 (segment (start 55.88 36.074) (end 59.436 39.63) (width 6) (layer "F.Cu") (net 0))
 (segment (start 52.578 39.376) (end 55.88 36.074) (width 6) (layer "F.Cu") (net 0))
 (segment (start 55.88 51.568) (end 59.436 55.124) (width 6) (layer "F.Cu") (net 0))
 (segment (start 52.578 54.87) (end 55.88 51.568) (width 6) (layer "F.Cu") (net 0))
 (segment (start 101.6 12.706) (end 105.156 16.262) (width 6) (layer "F.Cu") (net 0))
 (segment (start 98.298 16.008) (end 101.6 12.706) (width 6) (layer "F.Cu") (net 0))
 (segment (start 101.854 28.2) (end 105.41 31.756) (width 6) (layer "F.Cu") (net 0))
 (segment (start 98.552 31.502) (end 101.854 28.2) (width 6) (layer "F.Cu") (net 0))
 (segment (start 101.854 43.948) (end 105.41 47.504) (width 6) (layer "F.Cu") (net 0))
 (segment (start 98.552 47.25) (end 101.854 43.948) (width 6) (layer "F.Cu") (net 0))
 (segment (start 134.62 12.706) (end 138.176 16.262) (width 6) (layer "F.Cu") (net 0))
 (segment (start 131.318 16.008) (end 134.62 12.706) (width 6) (layer "F.Cu") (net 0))
 (segment (start 134.62 28.454) (end 138.176 32.01) (width 6) (layer "F.Cu") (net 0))
 (segment (start 131.318 31.756) (end 134.62 28.454) (width 6) (layer "F.Cu") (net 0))
 (segment (start 134.366 43.948) (end 137.922 47.504) (width 6) (layer "F.Cu") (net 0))
 (segment (start 131.064 47.25) (end 134.366 43.948) (width 6) (layer "F.Cu") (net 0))
 (segment (start 106.053599 38.374401) (end 105.966058 38.461942) (width 1) (layer "F.Cu") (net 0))
 (segment (start 149.948 37.592) (end 149.910216 37.629784) (width 1) (layer "F.Cu") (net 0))
 (segment (start 149.910216 41.821133) (end 145.649407 46.081942) (width 1) (layer "F.Cu") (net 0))
 (segment (start 127.762 3.81) (end 134.368 3.81) (width 6) (layer "F.Cu") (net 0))
 (segment (start 155.448 37.592) (end 155.448 42.248846) (width 1) (layer "F.Cu") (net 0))
 (segment (start 64.767397 53.752127) (end 64.563582 53.955942) (width 1) (layer "F.Cu") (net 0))
 (segment (start 149.948 19.057461) (end 146.09027 15.19973) (width 1) (layer "F.Cu") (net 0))
 (segment (start 152.428982 42.218832) (end 140.895687 53.752127) (width 1) (layer "F.Cu") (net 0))
 (segment (start 56.122 3.556) (end 60.39164 3.556) (width 4.13) (layer "F.Cu") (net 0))
 (segment (start 127.762 57.912) (end 134.516 57.912) (width 6) (layer "F.Cu") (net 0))
 (segment (start 105.966058 38.461942) (end 64.309582 38.461942) (width 1) (layer "F.Cu") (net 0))
 (segment (start 134.368 3.81) (end 134.622 3.556) (width 6) (layer "F.Cu") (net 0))
 (segment (start 147.669942 22.713942) (end 105.779942 22.713942) (width 1) (layer "F.Cu") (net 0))
 (segment (start 20.32 6.858) (end 23.622 3.556) (width 6) (layer "F.Cu") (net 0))
 (segment (start 60.39164 3.556) (end 64.309582 7.473942) (width 4.13) (layer "F.Cu") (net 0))
 (segment (start 158.712908 22.83521) (end 156.556118 24.992) (width 1) (layer "F.Cu") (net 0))
 (segment (start 155.448 20.792) (end 154.864137 20.792) (width 1) (layer "F.Cu") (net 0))
 (segment (start 134.698875 57.729125) (end 134.622 57.806) (width 1) (layer "F.Cu") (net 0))
 (segment (start 102.122 3.556) (end 109.22 3.556) (width 6) (layer "F.Cu") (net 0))
 (segment (start 154.864137 20.792) (end 141.54608 7.473942) (width 1) (layer "F.Cu") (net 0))
 (segment (start 143.603686 30.287838) (end 148.852162 30.287838) (width 1) (layer "F.Cu") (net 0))
 (segment (start 156.556118 24.992) (end 155.448 24.992) (width 1) (layer "F.Cu") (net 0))
 (segment (start 146.196058 15.093942) (end 143.303582 15.093942) (width 1) (layer "F.Cu") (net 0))
 (segment (start 158.712908 19.518861) (end 158.712908 22.83521) (width 1) (layer "F.Cu") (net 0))
 (segment (start 60.477525 11.306) (end 56.122 11.306) (width 4.13) (layer "F.Cu") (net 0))
 (segment (start 134.516 57.912) (end 134.622 57.806) (width 6) (layer "F.Cu") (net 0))
 (segment (start 152.428982 36.411018) (end 152.428982 42.218832) (width 1) (layer "F.Cu") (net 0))
 (segment (start 140.895687 53.752127) (end 64.767397 53.752127) (width 1) (layer "F.Cu") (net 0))
 (segment (start 134.622 3.556) (end 142.750047 3.556) (width 1) (layer "F.Cu") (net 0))
 (segment (start 141.54608 7.473942) (end 64.309582 7.473942) (width 1) (layer "F.Cu") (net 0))
 (segment (start 20.32 22.358) (end 23.622 19.056) (width 6) (layer "F.Cu") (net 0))
 (segment (start 139.967721 57.729125) (end 134.698875 57.729125) (width 1) (layer "F.Cu") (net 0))
 (segment (start 143.303582 30.587942) (end 143.603686 30.287838) (width 1) (layer "F.Cu") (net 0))
 (segment (start 109.114 57.806) (end 109.22 57.912) (width 6) (layer "F.Cu") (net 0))
 (segment (start 145.649407 46.081942) (end 143.049582 46.081942) (width 1) (layer "F.Cu") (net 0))
 (segment (start 144.965599 38.374401) (end 106.053599 38.374401) (width 1) (layer "F.Cu") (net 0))
 (segment (start 56.122 3.556) (end 56.122 11.306) (width 4.13) (layer "F.Cu") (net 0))
 (segment (start 23.622 3.556) (end 27.178 7.112) (width 6) (layer "F.Cu") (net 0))
 (segment (start 155.448 42.248846) (end 139.967721 57.729125) (width 1) (layer "F.Cu") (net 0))
 (segment (start 105.779942 22.713942) (end 64.309582 22.713942) (width 1) (layer "F.Cu") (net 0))
 (segment (start 149.948 24.992) (end 147.669942 22.713942) (width 1) (layer "F.Cu") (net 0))
 (segment (start 64.309582 7.473942) (end 60.477525 11.306) (width 4.13) (layer "F.Cu") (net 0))
 (segment (start 146.09027 15.19973) (end 146.196058 15.093942) (width 1) (layer "F.Cu") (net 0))
 (segment (start 148.852162 30.287838) (end 149.948 29.192) (width 1) (layer "F.Cu") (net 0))
 (segment (start 149.910216 37.629784) (end 149.910216 41.821133) (width 1) (layer "F.Cu") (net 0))
 (segment (start 149.948 20.792) (end 149.948 19.057461) (width 1) (layer "F.Cu") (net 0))
 (segment (start 23.622 19.056) (end 27.178 22.612) (width 6) (layer "F.Cu") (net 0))
 (segment (start 149.948 33.392) (end 144.965599 38.374401) (width 1) (layer "F.Cu") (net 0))
 (segment (start 142.750047 3.556) (end 158.712908 19.518861) (width 1) (layer "F.Cu") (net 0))
 (segment (start 102.122 57.806) (end 109.114 57.806) (width 6) (layer "F.Cu") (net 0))
 (segment (start 155.448 33.392) (end 152.428982 36.411018) (width 1) (layer "F.Cu") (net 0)))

